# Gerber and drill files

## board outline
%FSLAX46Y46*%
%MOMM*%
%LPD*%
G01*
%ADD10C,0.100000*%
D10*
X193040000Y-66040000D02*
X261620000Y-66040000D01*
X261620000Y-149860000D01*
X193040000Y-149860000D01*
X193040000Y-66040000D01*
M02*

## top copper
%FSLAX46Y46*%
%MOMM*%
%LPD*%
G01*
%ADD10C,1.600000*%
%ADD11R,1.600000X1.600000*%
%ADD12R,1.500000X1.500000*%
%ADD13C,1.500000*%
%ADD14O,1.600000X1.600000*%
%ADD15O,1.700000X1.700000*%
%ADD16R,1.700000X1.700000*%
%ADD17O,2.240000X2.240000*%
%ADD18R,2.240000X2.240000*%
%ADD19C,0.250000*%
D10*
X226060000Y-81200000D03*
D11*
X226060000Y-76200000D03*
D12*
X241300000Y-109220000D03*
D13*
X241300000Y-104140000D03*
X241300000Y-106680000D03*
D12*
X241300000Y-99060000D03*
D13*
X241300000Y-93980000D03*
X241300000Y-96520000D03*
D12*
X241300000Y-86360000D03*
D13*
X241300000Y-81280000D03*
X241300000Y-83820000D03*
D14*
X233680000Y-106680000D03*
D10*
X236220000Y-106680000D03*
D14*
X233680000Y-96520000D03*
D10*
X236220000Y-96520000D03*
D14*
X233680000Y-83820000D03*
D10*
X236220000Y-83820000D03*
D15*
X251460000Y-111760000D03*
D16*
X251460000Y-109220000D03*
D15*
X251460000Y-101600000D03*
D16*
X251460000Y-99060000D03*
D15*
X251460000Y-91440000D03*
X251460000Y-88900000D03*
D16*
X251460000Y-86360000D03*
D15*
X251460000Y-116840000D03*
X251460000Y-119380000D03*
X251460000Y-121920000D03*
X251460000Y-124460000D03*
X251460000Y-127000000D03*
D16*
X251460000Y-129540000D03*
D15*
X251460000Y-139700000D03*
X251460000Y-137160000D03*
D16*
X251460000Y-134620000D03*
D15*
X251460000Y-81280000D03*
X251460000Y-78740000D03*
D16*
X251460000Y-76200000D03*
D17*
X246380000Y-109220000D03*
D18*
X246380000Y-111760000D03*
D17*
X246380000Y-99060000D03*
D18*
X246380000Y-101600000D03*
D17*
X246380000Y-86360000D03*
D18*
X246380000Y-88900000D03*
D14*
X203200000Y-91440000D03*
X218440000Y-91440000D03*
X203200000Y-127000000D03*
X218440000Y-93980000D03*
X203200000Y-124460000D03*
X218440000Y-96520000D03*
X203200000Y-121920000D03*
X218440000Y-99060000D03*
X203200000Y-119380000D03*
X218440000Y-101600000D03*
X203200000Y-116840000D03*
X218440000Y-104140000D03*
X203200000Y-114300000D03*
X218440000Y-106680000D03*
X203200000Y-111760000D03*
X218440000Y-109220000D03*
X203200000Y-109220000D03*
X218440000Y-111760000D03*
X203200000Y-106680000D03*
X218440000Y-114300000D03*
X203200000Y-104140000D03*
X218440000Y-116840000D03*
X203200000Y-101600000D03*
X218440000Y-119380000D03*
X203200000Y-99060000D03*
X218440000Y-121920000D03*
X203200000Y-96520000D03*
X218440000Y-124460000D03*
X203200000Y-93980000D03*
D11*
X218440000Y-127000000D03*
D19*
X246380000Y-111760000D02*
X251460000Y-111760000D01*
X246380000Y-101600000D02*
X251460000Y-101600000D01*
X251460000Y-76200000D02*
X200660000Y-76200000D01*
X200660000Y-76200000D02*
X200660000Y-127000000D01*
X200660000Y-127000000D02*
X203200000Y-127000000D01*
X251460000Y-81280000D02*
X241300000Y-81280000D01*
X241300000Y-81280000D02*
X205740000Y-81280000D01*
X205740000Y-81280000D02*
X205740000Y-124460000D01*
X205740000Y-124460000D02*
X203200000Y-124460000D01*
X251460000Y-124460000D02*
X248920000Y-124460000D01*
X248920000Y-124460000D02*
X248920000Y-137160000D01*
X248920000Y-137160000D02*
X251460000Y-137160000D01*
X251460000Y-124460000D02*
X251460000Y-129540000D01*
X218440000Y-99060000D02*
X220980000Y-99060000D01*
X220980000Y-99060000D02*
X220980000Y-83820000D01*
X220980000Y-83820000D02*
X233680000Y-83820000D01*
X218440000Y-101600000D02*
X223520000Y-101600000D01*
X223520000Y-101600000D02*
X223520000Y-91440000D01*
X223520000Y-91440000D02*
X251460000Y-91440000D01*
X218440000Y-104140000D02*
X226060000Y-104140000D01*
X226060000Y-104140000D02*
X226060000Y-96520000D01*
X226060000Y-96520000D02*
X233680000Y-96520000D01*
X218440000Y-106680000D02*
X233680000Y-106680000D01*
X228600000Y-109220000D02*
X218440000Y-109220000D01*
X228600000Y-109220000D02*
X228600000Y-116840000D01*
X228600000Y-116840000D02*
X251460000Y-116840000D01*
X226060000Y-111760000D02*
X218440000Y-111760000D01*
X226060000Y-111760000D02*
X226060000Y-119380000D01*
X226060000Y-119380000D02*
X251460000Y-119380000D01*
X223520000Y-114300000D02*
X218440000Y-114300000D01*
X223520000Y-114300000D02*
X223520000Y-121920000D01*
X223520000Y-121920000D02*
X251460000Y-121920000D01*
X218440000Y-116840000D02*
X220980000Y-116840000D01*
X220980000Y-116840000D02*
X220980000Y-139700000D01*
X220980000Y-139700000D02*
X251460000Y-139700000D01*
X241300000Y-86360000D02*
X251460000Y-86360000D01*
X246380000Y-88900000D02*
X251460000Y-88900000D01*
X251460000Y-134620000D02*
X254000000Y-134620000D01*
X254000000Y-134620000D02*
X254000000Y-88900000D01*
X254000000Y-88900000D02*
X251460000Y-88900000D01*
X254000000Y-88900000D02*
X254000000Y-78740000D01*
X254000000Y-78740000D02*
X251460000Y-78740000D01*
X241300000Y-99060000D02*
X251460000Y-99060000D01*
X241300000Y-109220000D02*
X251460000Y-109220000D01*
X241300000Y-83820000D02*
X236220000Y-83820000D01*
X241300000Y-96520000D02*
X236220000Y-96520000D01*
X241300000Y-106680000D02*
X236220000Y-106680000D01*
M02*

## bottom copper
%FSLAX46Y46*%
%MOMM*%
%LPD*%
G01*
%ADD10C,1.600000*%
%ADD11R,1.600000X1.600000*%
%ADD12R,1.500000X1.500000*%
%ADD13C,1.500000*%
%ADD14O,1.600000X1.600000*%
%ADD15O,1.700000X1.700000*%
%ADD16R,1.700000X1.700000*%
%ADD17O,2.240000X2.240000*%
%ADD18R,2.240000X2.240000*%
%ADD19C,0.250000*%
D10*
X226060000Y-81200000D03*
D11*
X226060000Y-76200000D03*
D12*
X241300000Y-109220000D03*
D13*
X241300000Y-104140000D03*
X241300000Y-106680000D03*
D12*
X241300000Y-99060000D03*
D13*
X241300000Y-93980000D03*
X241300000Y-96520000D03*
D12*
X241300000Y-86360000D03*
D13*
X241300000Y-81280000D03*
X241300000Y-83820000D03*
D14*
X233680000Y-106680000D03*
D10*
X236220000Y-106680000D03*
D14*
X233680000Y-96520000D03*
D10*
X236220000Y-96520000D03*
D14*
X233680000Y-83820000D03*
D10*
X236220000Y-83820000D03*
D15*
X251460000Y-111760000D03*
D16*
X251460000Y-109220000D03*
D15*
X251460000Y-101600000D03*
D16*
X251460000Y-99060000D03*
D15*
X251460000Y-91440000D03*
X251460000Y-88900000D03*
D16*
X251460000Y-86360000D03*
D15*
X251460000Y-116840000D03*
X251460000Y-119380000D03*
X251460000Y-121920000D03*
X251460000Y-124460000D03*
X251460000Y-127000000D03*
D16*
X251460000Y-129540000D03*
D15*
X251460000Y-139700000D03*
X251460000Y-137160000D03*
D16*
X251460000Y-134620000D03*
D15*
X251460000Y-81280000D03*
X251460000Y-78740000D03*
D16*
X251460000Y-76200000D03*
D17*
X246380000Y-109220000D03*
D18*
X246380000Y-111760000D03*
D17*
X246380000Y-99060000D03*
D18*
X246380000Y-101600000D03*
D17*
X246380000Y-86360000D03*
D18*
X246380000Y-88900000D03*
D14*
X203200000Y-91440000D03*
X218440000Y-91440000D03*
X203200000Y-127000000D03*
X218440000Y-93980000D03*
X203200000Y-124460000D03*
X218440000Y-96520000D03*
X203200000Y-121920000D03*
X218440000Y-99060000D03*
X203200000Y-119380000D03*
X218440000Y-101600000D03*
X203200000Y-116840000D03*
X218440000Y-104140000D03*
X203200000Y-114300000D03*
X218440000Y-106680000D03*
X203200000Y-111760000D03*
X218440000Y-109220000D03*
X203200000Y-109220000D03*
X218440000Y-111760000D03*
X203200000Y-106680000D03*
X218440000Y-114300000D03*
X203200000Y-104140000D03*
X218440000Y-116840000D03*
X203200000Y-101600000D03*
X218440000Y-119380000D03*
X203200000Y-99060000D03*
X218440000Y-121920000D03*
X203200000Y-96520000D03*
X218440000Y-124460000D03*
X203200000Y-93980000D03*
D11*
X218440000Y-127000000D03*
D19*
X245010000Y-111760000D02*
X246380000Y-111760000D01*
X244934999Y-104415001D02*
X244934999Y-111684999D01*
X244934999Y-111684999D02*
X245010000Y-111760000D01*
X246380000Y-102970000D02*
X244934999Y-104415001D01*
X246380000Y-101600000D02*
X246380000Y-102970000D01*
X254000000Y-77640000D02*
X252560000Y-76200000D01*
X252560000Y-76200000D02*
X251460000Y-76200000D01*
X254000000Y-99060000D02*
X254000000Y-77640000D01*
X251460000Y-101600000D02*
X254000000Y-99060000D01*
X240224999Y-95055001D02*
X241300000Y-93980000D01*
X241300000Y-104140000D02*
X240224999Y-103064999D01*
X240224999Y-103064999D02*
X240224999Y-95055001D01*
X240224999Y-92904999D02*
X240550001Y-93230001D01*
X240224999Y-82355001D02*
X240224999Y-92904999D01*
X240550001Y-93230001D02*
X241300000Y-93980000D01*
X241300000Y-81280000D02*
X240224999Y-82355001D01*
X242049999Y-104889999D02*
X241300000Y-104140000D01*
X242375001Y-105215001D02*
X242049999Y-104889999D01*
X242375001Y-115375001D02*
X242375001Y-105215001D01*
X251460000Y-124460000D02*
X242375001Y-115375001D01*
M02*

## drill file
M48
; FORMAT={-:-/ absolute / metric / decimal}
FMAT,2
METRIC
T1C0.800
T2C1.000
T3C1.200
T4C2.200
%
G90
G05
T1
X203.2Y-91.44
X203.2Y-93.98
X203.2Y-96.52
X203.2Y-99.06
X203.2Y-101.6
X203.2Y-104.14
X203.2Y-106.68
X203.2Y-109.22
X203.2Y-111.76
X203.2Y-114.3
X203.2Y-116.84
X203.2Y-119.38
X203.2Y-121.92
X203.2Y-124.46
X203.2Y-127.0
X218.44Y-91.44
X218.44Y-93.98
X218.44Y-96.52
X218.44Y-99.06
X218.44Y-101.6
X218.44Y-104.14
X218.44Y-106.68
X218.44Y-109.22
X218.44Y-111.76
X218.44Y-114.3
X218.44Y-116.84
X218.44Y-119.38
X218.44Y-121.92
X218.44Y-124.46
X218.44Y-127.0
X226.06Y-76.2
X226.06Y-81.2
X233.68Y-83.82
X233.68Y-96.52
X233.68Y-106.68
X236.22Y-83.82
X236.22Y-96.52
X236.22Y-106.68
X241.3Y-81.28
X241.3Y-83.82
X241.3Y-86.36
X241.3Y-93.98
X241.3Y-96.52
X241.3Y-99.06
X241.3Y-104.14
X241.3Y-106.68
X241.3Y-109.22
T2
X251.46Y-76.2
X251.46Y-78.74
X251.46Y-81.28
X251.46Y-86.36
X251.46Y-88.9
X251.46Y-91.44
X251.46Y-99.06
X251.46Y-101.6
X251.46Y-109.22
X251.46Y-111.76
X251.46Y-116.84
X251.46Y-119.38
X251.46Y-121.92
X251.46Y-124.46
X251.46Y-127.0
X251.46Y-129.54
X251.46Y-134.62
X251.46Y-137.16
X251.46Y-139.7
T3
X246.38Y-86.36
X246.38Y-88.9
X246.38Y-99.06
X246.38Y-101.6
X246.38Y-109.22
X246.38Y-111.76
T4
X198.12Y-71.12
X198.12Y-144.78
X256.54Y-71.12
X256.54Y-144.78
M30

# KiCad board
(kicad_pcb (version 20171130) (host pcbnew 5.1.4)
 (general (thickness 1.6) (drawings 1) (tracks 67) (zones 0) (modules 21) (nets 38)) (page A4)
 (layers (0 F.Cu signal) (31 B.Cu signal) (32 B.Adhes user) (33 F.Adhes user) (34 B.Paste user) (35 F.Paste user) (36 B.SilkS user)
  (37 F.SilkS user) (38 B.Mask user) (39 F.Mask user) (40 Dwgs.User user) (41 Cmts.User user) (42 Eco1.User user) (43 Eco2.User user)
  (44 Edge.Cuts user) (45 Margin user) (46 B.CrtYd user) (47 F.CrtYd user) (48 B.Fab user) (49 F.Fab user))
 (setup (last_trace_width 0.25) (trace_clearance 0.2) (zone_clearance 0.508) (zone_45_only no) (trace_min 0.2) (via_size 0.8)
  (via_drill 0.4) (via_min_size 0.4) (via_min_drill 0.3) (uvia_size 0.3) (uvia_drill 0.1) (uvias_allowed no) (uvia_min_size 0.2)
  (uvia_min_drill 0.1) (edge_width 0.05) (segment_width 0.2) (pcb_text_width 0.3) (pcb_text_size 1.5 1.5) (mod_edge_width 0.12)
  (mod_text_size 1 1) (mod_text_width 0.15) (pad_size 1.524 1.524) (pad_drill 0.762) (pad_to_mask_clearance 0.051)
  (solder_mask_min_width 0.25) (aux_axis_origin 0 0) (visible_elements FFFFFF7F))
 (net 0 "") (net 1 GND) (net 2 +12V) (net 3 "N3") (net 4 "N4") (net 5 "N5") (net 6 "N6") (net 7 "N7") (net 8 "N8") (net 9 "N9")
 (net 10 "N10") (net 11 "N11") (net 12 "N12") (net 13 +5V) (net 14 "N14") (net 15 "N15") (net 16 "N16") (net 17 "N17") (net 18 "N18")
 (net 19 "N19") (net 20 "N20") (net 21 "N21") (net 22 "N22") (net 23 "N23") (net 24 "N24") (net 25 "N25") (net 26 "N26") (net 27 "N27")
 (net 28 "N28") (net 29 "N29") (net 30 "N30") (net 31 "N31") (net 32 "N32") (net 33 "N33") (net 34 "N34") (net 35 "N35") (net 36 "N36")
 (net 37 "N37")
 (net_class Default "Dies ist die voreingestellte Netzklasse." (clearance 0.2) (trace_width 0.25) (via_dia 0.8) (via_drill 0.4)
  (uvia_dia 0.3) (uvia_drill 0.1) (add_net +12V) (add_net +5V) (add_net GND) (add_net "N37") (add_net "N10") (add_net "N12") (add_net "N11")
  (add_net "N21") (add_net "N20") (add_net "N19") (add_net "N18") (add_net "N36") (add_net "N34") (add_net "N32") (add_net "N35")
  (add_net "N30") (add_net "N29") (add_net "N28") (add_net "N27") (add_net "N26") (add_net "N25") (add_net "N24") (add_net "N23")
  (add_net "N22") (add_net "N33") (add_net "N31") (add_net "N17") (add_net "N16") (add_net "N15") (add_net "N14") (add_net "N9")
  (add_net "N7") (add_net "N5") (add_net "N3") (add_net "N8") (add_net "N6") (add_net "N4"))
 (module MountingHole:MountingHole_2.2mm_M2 (layer F.Cu) (at 198.12 71.12)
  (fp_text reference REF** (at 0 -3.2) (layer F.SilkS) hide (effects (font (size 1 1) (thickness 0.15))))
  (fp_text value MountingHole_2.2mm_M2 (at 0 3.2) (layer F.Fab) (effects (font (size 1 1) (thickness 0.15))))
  (pad 1 np_thru_hole circle (at 0 0) (size 2.2 2.2) (drill 2.2) (layers *.Cu *.Mask)))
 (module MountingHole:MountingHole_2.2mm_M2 (layer F.Cu) (at 198.12 144.78)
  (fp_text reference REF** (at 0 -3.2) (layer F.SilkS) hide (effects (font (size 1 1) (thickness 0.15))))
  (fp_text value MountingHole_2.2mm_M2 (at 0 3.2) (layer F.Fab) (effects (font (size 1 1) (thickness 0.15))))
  (pad 1 np_thru_hole circle (at 0 0) (size 2.2 2.2) (drill 2.2) (layers *.Cu *.Mask)))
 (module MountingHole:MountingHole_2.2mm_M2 (layer F.Cu) (at 256.54 144.78)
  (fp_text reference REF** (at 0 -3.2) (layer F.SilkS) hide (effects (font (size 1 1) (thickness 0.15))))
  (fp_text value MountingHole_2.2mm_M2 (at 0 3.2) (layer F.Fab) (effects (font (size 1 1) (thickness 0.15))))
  (pad 1 np_thru_hole circle (at 0 0) (size 2.2 2.2) (drill 2.2) (layers *.Cu *.Mask)))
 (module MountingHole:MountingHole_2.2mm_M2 (layer F.Cu) (at 256.54 71.12)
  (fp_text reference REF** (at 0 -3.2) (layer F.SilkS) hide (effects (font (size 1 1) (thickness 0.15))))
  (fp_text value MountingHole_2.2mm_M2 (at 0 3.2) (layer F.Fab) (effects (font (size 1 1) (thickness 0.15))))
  (pad 1 np_thru_hole circle (at 0 0) (size 2.2 2.2) (drill 2.2) (layers *.Cu *.Mask)))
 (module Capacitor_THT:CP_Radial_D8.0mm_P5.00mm (layer F.Cu) (at 226.06 76.2 270)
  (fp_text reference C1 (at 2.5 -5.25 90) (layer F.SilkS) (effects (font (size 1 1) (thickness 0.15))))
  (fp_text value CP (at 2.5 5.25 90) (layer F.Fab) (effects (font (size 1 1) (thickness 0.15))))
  (pad 2 thru_hole circle (at 5 0 270) (size 1.6 1.6) (drill 0.8) (layers *.Cu *.Mask) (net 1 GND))
  (pad 1 thru_hole rect (at 0 0 270) (size 1.6 1.6) (drill 0.8) (layers *.Cu *.Mask) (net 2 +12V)))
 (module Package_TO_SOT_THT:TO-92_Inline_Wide (layer F.Cu) (at 241.3 109.22 90)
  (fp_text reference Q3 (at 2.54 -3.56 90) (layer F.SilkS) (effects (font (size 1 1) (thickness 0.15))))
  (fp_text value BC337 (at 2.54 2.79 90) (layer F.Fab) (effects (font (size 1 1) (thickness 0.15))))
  (pad 1 thru_hole rect (at 0 0 180) (size 1.5 1.5) (drill 0.8) (layers *.Cu *.Mask) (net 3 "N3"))
  (pad 3 thru_hole circle (at 5.08 0 180) (size 1.5 1.5) (drill 0.8) (layers *.Cu *.Mask) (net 1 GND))
  (pad 2 thru_hole circle (at 2.54 0 180) (size 1.5 1.5) (drill 0.8) (layers *.Cu *.Mask) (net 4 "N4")))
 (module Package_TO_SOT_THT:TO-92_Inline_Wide (layer F.Cu) (at 241.3 99.06 90)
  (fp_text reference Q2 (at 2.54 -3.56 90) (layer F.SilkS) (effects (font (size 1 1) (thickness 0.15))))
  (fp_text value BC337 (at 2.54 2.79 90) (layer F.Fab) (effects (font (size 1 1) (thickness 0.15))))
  (pad 1 thru_hole rect (at 0 0 180) (size 1.5 1.5) (drill 0.8) (layers *.Cu *.Mask) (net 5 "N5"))
  (pad 3 thru_hole circle (at 5.08 0 180) (size 1.5 1.5) (drill 0.8) (layers *.Cu *.Mask) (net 1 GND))
  (pad 2 thru_hole circle (at 2.54 0 180) (size 1.5 1.5) (drill 0.8) (layers *.Cu *.Mask) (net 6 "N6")))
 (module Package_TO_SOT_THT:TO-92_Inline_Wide (layer F.Cu) (at 241.3 86.36 90)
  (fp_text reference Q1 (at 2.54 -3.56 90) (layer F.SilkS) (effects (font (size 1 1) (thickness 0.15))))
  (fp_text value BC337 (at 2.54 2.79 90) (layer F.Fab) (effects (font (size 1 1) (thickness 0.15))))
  (pad 1 thru_hole rect (at 0 0 180) (size 1.5 1.5) (drill 0.8) (layers *.Cu *.Mask) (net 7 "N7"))
  (pad 3 thru_hole circle (at 5.08 0 180) (size 1.5 1.5) (drill 0.8) (layers *.Cu *.Mask) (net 1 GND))
  (pad 2 thru_hole circle (at 2.54 0 180) (size 1.5 1.5) (drill 0.8) (layers *.Cu *.Mask) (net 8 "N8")))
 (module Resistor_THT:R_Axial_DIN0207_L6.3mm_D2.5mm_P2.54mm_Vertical (layer F.Cu) (at 236.22 106.68 180)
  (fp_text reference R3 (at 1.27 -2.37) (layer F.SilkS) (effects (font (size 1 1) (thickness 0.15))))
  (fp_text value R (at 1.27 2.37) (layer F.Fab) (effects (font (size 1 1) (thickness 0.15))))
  (pad 2 thru_hole oval (at 2.54 0 180) (size 1.6 1.6) (drill 0.8) (layers *.Cu *.Mask) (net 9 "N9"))
  (pad 1 thru_hole circle (at 0 0 180) (size 1.6 1.6) (drill 0.8) (layers *.Cu *.Mask) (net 4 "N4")))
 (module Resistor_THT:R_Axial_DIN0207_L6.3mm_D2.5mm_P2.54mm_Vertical (layer F.Cu) (at 236.22 96.52 180)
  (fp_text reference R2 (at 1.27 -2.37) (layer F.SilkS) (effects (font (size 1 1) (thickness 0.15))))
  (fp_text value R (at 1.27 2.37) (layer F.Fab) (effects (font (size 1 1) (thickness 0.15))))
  (pad 2 thru_hole oval (at 2.54 0 180) (size 1.6 1.6) (drill 0.8) (layers *.Cu *.Mask) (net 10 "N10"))
  (pad 1 thru_hole circle (at 0 0 180) (size 1.6 1.6) (drill 0.8) (layers *.Cu *.Mask) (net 6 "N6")))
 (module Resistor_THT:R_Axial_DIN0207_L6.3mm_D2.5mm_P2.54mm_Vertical (layer F.Cu) (at 236.22 83.82 180)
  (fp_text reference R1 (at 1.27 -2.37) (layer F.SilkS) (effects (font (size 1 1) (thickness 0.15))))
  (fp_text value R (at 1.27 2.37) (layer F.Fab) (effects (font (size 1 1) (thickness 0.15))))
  (pad 2 thru_hole oval (at 2.54 0 180) (size 1.6 1.6) (drill 0.8) (layers *.Cu *.Mask) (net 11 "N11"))
  (pad 1 thru_hole circle (at 0 0 180) (size 1.6 1.6) (drill 0.8) (layers *.Cu *.Mask) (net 8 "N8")))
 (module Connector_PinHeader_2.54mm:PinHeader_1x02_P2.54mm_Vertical (layer F.Cu) (at 251.46 109.22)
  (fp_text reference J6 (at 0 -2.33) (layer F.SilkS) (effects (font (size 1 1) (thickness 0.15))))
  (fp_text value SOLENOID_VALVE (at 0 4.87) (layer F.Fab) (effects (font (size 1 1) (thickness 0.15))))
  (pad 2 thru_hole oval (at 0 2.54) (size 1.7 1.7) (drill 1) (layers *.Cu *.Mask) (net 2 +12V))
  (pad 1 thru_hole rect (at 0 0) (size 1.7 1.7) (drill 1) (layers *.Cu *.Mask) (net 3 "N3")))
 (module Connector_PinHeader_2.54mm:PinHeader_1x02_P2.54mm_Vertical (layer F.Cu) (at 251.46 99.06)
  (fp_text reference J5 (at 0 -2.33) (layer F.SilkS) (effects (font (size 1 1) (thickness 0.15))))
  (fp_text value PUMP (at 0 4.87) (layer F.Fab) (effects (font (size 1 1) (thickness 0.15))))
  (pad 2 thru_hole oval (at 0 2.54) (size 1.7 1.7) (drill 1) (layers *.Cu *.Mask) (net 2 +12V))
  (pad 1 thru_hole rect (at 0 0) (size 1.7 1.7) (drill 1) (layers *.Cu *.Mask) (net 5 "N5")))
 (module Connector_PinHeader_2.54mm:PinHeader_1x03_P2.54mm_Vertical (layer F.Cu) (at 251.46 86.36)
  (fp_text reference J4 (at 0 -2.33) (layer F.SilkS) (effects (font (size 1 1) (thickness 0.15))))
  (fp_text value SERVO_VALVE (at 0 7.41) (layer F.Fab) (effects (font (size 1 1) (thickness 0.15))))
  (pad 3 thru_hole oval (at 0 5.08) (size 1.7 1.7) (drill 1) (layers *.Cu *.Mask) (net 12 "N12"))
  (pad 2 thru_hole oval (at 0 2.54) (size 1.7 1.7) (drill 1) (layers *.Cu *.Mask) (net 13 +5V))
  (pad 1 thru_hole rect (at 0 0) (size 1.7 1.7) (drill 1) (layers *.Cu *.Mask) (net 7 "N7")))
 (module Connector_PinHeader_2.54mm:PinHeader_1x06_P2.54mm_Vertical (layer F.Cu) (at 251.46 129.54 180)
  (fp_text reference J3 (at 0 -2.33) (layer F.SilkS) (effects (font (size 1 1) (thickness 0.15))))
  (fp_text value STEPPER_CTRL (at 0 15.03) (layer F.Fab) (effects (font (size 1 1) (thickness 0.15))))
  (pad 6 thru_hole oval (at 0 12.7 180) (size 1.7 1.7) (drill 1) (layers *.Cu *.Mask) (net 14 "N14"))
  (pad 5 thru_hole oval (at 0 10.16 180) (size 1.7 1.7) (drill 1) (layers *.Cu *.Mask) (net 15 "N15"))
  (pad 4 thru_hole oval (at 0 7.62 180) (size 1.7 1.7) (drill 1) (layers *.Cu *.Mask) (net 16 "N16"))
  (pad 3 thru_hole oval (at 0 5.08 180) (size 1.7 1.7) (drill 1) (layers *.Cu *.Mask) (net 1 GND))
  (pad 2 thru_hole oval (at 0 2.54 180) (size 1.7 1.7) (drill 1) (layers *.Cu *.Mask) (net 1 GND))
  (pad 1 thru_hole rect (at 0 0 180) (size 1.7 1.7) (drill 1) (layers *.Cu *.Mask) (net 1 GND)))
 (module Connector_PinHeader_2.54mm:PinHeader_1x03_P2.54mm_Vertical (layer F.Cu) (at 251.46 134.62)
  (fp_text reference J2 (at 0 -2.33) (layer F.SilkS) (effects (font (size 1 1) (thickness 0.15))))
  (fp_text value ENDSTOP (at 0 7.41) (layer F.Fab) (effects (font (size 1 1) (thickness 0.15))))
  (pad 3 thru_hole oval (at 0 5.08) (size 1.7 1.7) (drill 1) (layers *.Cu *.Mask) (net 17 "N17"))
  (pad 2 thru_hole oval (at 0 2.54) (size 1.7 1.7) (drill 1) (layers *.Cu *.Mask) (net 1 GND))
  (pad 1 thru_hole rect (at 0 0) (size 1.7 1.7) (drill 1) (layers *.Cu *.Mask) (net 13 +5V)))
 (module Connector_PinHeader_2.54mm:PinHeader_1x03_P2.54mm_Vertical (layer F.Cu) (at 251.46 76.2)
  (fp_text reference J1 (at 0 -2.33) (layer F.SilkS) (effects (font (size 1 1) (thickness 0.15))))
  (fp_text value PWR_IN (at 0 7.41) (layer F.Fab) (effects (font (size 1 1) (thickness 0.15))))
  (pad 3 thru_hole oval (at 0 5.08) (size 1.7 1.7) (drill 1) (layers *.Cu *.Mask) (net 1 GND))
  (pad 2 thru_hole oval (at 0 2.54) (size 1.7 1.7) (drill 1) (layers *.Cu *.Mask) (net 13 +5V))
  (pad 1 thru_hole rect (at 0 0) (size 1.7 1.7) (drill 1) (layers *.Cu *.Mask) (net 2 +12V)))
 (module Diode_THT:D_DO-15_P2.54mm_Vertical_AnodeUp (layer F.Cu) (at 246.38 111.76 90)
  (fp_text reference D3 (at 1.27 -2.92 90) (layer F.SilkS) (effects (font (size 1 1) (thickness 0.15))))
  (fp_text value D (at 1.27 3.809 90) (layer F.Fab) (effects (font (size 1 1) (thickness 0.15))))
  (pad 2 thru_hole oval (at 2.54 0 90) (size 2.24 2.24) (drill 1.2) (layers *.Cu *.Mask) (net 3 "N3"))
  (pad 1 thru_hole rect (at 0 0 90) (size 2.24 2.24) (drill 1.2) (layers *.Cu *.Mask) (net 2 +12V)))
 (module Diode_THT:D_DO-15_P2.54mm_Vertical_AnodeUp (layer F.Cu) (at 246.38 101.6 90)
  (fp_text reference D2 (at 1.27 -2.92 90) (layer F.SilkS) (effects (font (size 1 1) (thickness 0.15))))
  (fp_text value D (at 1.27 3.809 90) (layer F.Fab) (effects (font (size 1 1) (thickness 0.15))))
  (pad 2 thru_hole oval (at 2.54 0 90) (size 2.24 2.24) (drill 1.2) (layers *.Cu *.Mask) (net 5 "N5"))
  (pad 1 thru_hole rect (at 0 0 90) (size 2.24 2.24) (drill 1.2) (layers *.Cu *.Mask) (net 2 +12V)))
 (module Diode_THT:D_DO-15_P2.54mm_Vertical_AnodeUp (layer F.Cu) (at 246.38 88.9 90)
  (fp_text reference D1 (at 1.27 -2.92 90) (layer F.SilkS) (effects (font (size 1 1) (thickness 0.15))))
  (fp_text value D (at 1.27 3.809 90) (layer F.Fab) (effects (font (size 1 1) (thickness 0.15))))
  (pad 2 thru_hole oval (at 2.54 0 90) (size 2.24 2.24) (drill 1.2) (layers *.Cu *.Mask) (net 7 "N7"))
  (pad 1 thru_hole rect (at 0 0 90) (size 2.24 2.24) (drill 1.2) (layers *.Cu *.Mask) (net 13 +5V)))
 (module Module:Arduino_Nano (layer F.Cu) (at 218.44 127 180)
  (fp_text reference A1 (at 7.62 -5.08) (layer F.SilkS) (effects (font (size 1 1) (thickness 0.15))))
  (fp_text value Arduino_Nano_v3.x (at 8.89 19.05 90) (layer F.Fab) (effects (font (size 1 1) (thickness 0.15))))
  (pad 16 thru_hole oval (at 15.24 35.56 180) (size 1.6 1.6) (drill 0.8) (layers *.Cu *.Mask) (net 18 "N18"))
  (pad 15 thru_hole oval (at 0 35.56 180) (size 1.6 1.6) (drill 0.8) (layers *.Cu *.Mask) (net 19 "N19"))
  (pad 30 thru_hole oval (at 15.24 0 180) (size 1.6 1.6) (drill 0.8) (layers *.Cu *.Mask) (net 2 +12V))
  (pad 14 thru_hole oval (at 0 33.02 180) (size 1.6 1.6) (drill 0.8) (layers *.Cu *.Mask) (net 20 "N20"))
  (pad 29 thru_hole oval (at 15.24 2.54 180) (size 1.6 1.6) (drill 0.8) (layers *.Cu *.Mask) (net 1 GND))
  (pad 13 thru_hole oval (at 0 30.48 180) (size 1.6 1.6) (drill 0.8) (layers *.Cu *.Mask) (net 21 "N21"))
  (pad 28 thru_hole oval (at 15.24 5.08 180) (size 1.6 1.6) (drill 0.8) (layers *.Cu *.Mask) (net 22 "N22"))
  (pad 12 thru_hole oval (at 0 27.94 180) (size 1.6 1.6) (drill 0.8) (layers *.Cu *.Mask) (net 11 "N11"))
  (pad 27 thru_hole oval (at 15.24 7.62 180) (size 1.6 1.6) (drill 0.8) (layers *.Cu *.Mask) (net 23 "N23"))
  (pad 11 thru_hole oval (at 0 25.4 180) (size 1.6 1.6) (drill 0.8) (layers *.Cu *.Mask) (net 12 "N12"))
  (pad 26 thru_hole oval (at 15.24 10.16 180) (size 1.6 1.6) (drill 0.8) (layers *.Cu *.Mask) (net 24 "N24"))
  (pad 10 thru_hole oval (at 0 22.86 180) (size 1.6 1.6) (drill 0.8) (layers *.Cu *.Mask) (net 10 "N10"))
  (pad 25 thru_hole oval (at 15.24 12.7 180) (size 1.6 1.6) (drill 0.8) (layers *.Cu *.Mask) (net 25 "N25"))
  (pad 9 thru_hole oval (at 0 20.32 180) (size 1.6 1.6) (drill 0.8) (layers *.Cu *.Mask) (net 9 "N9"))
  (pad 24 thru_hole oval (at 15.24 15.24 180) (size 1.6 1.6) (drill 0.8) (layers *.Cu *.Mask) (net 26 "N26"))
  (pad 8 thru_hole oval (at 0 17.78 180) (size 1.6 1.6) (drill 0.8) (layers *.Cu *.Mask) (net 14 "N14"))
  (pad 23 thru_hole oval (at 15.24 17.78 180) (size 1.6 1.6) (drill 0.8) (layers *.Cu *.Mask) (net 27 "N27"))
  (pad 7 thru_hole oval (at 0 15.24 180) (size 1.6 1.6) (drill 0.8) (layers *.Cu *.Mask) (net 15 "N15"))
  (pad 22 thru_hole oval (at 15.24 20.32 180) (size 1.6 1.6) (drill 0.8) (layers *.Cu *.Mask) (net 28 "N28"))
  (pad 6 thru_hole oval (at 0 12.7 180) (size 1.6 1.6) (drill 0.8) (layers *.Cu *.Mask) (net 16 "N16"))
  (pad 21 thru_hole oval (at 15.24 22.86 180) (size 1.6 1.6) (drill 0.8) (layers *.Cu *.Mask) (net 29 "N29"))
  (pad 5 thru_hole oval (at 0 10.16 180) (size 1.6 1.6) (drill 0.8) (layers *.Cu *.Mask) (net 17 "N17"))
  (pad 20 thru_hole oval (at 15.24 25.4 180) (size 1.6 1.6) (drill 0.8) (layers *.Cu *.Mask) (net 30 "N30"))
  (pad 4 thru_hole oval (at 0 7.62 180) (size 1.6 1.6) (drill 0.8) (layers *.Cu *.Mask) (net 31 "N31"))
  (pad 19 thru_hole oval (at 15.24 27.94 180) (size 1.6 1.6) (drill 0.8) (layers *.Cu *.Mask) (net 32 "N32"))
  (pad 3 thru_hole oval (at 0 5.08 180) (size 1.6 1.6) (drill 0.8) (layers *.Cu *.Mask) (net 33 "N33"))
  (pad 18 thru_hole oval (at 15.24 30.48 180) (size 1.6 1.6) (drill 0.8) (layers *.Cu *.Mask) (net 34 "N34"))
  (pad 2 thru_hole oval (at 0 2.54 180) (size 1.6 1.6) (drill 0.8) (layers *.Cu *.Mask) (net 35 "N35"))
  (pad 17 thru_hole oval (at 15.24 33.02 180) (size 1.6 1.6) (drill 0.8) (layers *.Cu *.Mask) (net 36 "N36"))
  (pad 1 thru_hole rect (at 0 0 180) (size 1.6 1.6) (drill 0.8) (layers *.Cu *.Mask) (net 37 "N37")))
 (gr_poly (pts (xy 193.04 66.04) (xy 261.62 66.04) (xy 261.62 149.86) (xy 193.04 149.86)) (layer Edge.Cuts) (width 0.1))
 (segment (start 246.38 111.76) (end 251.46 111.76) (width 0.25) (layer F.Cu) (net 2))
 (segment (start 246.38 101.6) (end 251.46 101.6) (width 0.25) (layer F.Cu) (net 2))
 (segment (start 251.46 76.2) (end 200.66 76.2) (width 0.25) (layer F.Cu) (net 2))
 (segment (start 200.66 76.2) (end 200.66 127) (width 0.25) (layer F.Cu) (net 2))
 (segment (start 200.66 127) (end 203.2 127) (width 0.25) (layer F.Cu) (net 2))
 (segment (start 245.01 111.76) (end 246.38 111.76) (width 0.25) (layer B.Cu) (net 2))
 (segment (start 244.934999 104.415001) (end 244.934999 111.684999) (width 0.25) (layer B.Cu) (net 2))
 (segment (start 244.934999 111.684999) (end 245.01 111.76) (width 0.25) (layer B.Cu) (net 2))
 (segment (start 246.38 102.97) (end 244.934999 104.415001) (width 0.25) (layer B.Cu) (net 2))
 (segment (start 246.38 101.6) (end 246.38 102.97) (width 0.25) (layer B.Cu) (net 2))
 (segment (start 254 77.64) (end 252.56 76.2) (width 0.25) (layer B.Cu) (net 2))
 (segment (start 252.56 76.2) (end 251.46 76.2) (width 0.25) (layer B.Cu) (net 2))
 (segment (start 254 99.06) (end 254 77.64) (width 0.25) (layer B.Cu) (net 2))
 (segment (start 251.46 101.6) (end 254 99.06) (width 0.25) (layer B.Cu) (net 2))
 (segment (start 251.46 81.28) (end 241.3 81.28) (width 0.25) (layer F.Cu) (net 1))
 (segment (start 241.3 81.28) (end 205.74 81.28) (width 0.25) (layer F.Cu) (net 1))
 (segment (start 205.74 81.28) (end 205.74 124.46) (width 0.25) (layer F.Cu) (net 1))
 (segment (start 205.74 124.46) (end 203.2 124.46) (width 0.25) (layer F.Cu) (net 1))
 (segment (start 240.224999 95.055001) (end 241.3 93.98) (width 0.25) (layer B.Cu) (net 1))
 (segment (start 241.3 104.14) (end 240.224999 103.064999) (width 0.25) (layer B.Cu) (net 1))
 (segment (start 240.224999 103.064999) (end 240.224999 95.055001) (width 0.25) (layer B.Cu) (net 1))
 (segment (start 240.224999 92.904999) (end 240.550001 93.230001) (width 0.25) (layer B.Cu) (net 1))
 (segment (start 240.224999 82.355001) (end 240.224999 92.904999) (width 0.25) (layer B.Cu) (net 1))
 (segment (start 240.550001 93.230001) (end 241.3 93.98) (width 0.25) (layer B.Cu) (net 1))
 (segment (start 241.3 81.28) (end 240.224999 82.355001) (width 0.25) (layer B.Cu) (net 1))
 (segment (start 251.46 124.46) (end 248.92 124.46) (width 0.25) (layer F.Cu) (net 1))
 (segment (start 248.92 124.46) (end 248.92 137.16) (width 0.25) (layer F.Cu) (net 1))
 (segment (start 248.92 137.16) (end 251.46 137.16) (width 0.25) (layer F.Cu) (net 1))
 (segment (start 251.46 124.46) (end 251.46 129.54) (width 0.25) (layer F.Cu) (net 1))
 (segment (start 242.049999 104.889999) (end 241.3 104.14) (width 0.25) (layer B.Cu) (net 1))
 (segment (start 242.375001 105.215001) (end 242.049999 104.889999) (width 0.25) (layer B.Cu) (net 1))
 (segment (start 242.375001 115.375001) (end 242.375001 105.215001) (width 0.25) (layer B.Cu) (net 1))
 (segment (start 251.46 124.46) (end 242.375001 115.375001) (width 0.25) (layer B.Cu) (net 1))
 (segment (start 218.44 99.06) (end 220.98 99.06) (width 0.25) (layer F.Cu) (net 11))
 (segment (start 220.98 99.06) (end 220.98 83.82) (width 0.25) (layer F.Cu) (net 11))
 (segment (start 220.98 83.82) (end 233.68 83.82) (width 0.25) (layer F.Cu) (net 11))
 (segment (start 218.44 101.6) (end 223.52 101.6) (width 0.25) (layer F.Cu) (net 12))
 (segment (start 223.52 101.6) (end 223.52 91.44) (width 0.25) (layer F.Cu) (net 12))
 (segment (start 223.52 91.44) (end 251.46 91.44) (width 0.25) (layer F.Cu) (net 12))
 (segment (start 218.44 104.14) (end 226.06 104.14) (width 0.25) (layer F.Cu) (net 10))
 (segment (start 226.06 104.14) (end 226.06 96.52) (width 0.25) (layer F.Cu) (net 10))
 (segment (start 226.06 96.52) (end 233.68 96.52) (width 0.25) (layer F.Cu) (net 10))
 (segment (start 218.44 106.68) (end 233.68 106.68) (width 0.25) (layer F.Cu) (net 9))
 (segment (start 228.6 109.22) (end 218.44 109.22) (width 0.25) (layer F.Cu) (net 14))
 (segment (start 228.6 109.22) (end 228.6 116.84) (width 0.25) (layer F.Cu) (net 14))
 (segment (start 228.6 116.84) (end 251.46 116.84) (width 0.25) (layer F.Cu) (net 14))
 (segment (start 226.06 111.76) (end 218.44 111.76) (width 0.25) (layer F.Cu) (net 15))
 (segment (start 226.06 111.76) (end 226.06 119.38) (width 0.25) (layer F.Cu) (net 15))
 (segment (start 226.06 119.38) (end 251.46 119.38) (width 0.25) (layer F.Cu) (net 15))
 (segment (start 223.52 114.3) (end 218.44 114.3) (width 0.25) (layer F.Cu) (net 16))
 (segment (start 223.52 114.3) (end 223.52 121.92) (width 0.25) (layer F.Cu) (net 16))
 (segment (start 223.52 121.92) (end 251.46 121.92) (width 0.25) (layer F.Cu) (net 16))
 (segment (start 218.44 116.84) (end 220.98 116.84) (width 0.25) (layer F.Cu) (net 17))
 (segment (start 220.98 116.84) (end 220.98 139.7) (width 0.25) (layer F.Cu) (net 17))
 (segment (start 220.98 139.7) (end 251.46 139.7) (width 0.25) (layer F.Cu) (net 17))
 (segment (start 241.3 86.36) (end 251.46 86.36) (width 0.25) (layer F.Cu) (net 7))
 (segment (start 246.38 88.9) (end 251.46 88.9) (width 0.25) (layer F.Cu) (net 13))
 (segment (start 251.46 134.62) (end 254 134.62) (width 0.25) (layer F.Cu) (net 13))
 (segment (start 254 134.62) (end 254 88.9) (width 0.25) (layer F.Cu) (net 13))
 (segment (start 254 88.9) (end 251.46 88.9) (width 0.25) (layer F.Cu) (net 13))
 (segment (start 254 88.9) (end 254 78.74) (width 0.25) (layer F.Cu) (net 13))
 (segment (start 254 78.74) (end 251.46 78.74) (width 0.25) (layer F.Cu) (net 13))
 (segment (start 241.3 99.06) (end 251.46 99.06) (width 0.25) (layer F.Cu) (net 5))
 (segment (start 241.3 109.22) (end 251.46 109.22) (width 0.25) (layer F.Cu) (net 3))
 (segment (start 241.3 83.82) (end 236.22 83.82) (width 0.25) (layer F.Cu) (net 8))
 (segment (start 241.3 96.52) (end 236.22 96.52) (width 0.25) (layer F.Cu) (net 6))
 (segment (start 241.3 106.68) (end 236.22 106.68) (width 0.25) (layer F.Cu) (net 4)))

